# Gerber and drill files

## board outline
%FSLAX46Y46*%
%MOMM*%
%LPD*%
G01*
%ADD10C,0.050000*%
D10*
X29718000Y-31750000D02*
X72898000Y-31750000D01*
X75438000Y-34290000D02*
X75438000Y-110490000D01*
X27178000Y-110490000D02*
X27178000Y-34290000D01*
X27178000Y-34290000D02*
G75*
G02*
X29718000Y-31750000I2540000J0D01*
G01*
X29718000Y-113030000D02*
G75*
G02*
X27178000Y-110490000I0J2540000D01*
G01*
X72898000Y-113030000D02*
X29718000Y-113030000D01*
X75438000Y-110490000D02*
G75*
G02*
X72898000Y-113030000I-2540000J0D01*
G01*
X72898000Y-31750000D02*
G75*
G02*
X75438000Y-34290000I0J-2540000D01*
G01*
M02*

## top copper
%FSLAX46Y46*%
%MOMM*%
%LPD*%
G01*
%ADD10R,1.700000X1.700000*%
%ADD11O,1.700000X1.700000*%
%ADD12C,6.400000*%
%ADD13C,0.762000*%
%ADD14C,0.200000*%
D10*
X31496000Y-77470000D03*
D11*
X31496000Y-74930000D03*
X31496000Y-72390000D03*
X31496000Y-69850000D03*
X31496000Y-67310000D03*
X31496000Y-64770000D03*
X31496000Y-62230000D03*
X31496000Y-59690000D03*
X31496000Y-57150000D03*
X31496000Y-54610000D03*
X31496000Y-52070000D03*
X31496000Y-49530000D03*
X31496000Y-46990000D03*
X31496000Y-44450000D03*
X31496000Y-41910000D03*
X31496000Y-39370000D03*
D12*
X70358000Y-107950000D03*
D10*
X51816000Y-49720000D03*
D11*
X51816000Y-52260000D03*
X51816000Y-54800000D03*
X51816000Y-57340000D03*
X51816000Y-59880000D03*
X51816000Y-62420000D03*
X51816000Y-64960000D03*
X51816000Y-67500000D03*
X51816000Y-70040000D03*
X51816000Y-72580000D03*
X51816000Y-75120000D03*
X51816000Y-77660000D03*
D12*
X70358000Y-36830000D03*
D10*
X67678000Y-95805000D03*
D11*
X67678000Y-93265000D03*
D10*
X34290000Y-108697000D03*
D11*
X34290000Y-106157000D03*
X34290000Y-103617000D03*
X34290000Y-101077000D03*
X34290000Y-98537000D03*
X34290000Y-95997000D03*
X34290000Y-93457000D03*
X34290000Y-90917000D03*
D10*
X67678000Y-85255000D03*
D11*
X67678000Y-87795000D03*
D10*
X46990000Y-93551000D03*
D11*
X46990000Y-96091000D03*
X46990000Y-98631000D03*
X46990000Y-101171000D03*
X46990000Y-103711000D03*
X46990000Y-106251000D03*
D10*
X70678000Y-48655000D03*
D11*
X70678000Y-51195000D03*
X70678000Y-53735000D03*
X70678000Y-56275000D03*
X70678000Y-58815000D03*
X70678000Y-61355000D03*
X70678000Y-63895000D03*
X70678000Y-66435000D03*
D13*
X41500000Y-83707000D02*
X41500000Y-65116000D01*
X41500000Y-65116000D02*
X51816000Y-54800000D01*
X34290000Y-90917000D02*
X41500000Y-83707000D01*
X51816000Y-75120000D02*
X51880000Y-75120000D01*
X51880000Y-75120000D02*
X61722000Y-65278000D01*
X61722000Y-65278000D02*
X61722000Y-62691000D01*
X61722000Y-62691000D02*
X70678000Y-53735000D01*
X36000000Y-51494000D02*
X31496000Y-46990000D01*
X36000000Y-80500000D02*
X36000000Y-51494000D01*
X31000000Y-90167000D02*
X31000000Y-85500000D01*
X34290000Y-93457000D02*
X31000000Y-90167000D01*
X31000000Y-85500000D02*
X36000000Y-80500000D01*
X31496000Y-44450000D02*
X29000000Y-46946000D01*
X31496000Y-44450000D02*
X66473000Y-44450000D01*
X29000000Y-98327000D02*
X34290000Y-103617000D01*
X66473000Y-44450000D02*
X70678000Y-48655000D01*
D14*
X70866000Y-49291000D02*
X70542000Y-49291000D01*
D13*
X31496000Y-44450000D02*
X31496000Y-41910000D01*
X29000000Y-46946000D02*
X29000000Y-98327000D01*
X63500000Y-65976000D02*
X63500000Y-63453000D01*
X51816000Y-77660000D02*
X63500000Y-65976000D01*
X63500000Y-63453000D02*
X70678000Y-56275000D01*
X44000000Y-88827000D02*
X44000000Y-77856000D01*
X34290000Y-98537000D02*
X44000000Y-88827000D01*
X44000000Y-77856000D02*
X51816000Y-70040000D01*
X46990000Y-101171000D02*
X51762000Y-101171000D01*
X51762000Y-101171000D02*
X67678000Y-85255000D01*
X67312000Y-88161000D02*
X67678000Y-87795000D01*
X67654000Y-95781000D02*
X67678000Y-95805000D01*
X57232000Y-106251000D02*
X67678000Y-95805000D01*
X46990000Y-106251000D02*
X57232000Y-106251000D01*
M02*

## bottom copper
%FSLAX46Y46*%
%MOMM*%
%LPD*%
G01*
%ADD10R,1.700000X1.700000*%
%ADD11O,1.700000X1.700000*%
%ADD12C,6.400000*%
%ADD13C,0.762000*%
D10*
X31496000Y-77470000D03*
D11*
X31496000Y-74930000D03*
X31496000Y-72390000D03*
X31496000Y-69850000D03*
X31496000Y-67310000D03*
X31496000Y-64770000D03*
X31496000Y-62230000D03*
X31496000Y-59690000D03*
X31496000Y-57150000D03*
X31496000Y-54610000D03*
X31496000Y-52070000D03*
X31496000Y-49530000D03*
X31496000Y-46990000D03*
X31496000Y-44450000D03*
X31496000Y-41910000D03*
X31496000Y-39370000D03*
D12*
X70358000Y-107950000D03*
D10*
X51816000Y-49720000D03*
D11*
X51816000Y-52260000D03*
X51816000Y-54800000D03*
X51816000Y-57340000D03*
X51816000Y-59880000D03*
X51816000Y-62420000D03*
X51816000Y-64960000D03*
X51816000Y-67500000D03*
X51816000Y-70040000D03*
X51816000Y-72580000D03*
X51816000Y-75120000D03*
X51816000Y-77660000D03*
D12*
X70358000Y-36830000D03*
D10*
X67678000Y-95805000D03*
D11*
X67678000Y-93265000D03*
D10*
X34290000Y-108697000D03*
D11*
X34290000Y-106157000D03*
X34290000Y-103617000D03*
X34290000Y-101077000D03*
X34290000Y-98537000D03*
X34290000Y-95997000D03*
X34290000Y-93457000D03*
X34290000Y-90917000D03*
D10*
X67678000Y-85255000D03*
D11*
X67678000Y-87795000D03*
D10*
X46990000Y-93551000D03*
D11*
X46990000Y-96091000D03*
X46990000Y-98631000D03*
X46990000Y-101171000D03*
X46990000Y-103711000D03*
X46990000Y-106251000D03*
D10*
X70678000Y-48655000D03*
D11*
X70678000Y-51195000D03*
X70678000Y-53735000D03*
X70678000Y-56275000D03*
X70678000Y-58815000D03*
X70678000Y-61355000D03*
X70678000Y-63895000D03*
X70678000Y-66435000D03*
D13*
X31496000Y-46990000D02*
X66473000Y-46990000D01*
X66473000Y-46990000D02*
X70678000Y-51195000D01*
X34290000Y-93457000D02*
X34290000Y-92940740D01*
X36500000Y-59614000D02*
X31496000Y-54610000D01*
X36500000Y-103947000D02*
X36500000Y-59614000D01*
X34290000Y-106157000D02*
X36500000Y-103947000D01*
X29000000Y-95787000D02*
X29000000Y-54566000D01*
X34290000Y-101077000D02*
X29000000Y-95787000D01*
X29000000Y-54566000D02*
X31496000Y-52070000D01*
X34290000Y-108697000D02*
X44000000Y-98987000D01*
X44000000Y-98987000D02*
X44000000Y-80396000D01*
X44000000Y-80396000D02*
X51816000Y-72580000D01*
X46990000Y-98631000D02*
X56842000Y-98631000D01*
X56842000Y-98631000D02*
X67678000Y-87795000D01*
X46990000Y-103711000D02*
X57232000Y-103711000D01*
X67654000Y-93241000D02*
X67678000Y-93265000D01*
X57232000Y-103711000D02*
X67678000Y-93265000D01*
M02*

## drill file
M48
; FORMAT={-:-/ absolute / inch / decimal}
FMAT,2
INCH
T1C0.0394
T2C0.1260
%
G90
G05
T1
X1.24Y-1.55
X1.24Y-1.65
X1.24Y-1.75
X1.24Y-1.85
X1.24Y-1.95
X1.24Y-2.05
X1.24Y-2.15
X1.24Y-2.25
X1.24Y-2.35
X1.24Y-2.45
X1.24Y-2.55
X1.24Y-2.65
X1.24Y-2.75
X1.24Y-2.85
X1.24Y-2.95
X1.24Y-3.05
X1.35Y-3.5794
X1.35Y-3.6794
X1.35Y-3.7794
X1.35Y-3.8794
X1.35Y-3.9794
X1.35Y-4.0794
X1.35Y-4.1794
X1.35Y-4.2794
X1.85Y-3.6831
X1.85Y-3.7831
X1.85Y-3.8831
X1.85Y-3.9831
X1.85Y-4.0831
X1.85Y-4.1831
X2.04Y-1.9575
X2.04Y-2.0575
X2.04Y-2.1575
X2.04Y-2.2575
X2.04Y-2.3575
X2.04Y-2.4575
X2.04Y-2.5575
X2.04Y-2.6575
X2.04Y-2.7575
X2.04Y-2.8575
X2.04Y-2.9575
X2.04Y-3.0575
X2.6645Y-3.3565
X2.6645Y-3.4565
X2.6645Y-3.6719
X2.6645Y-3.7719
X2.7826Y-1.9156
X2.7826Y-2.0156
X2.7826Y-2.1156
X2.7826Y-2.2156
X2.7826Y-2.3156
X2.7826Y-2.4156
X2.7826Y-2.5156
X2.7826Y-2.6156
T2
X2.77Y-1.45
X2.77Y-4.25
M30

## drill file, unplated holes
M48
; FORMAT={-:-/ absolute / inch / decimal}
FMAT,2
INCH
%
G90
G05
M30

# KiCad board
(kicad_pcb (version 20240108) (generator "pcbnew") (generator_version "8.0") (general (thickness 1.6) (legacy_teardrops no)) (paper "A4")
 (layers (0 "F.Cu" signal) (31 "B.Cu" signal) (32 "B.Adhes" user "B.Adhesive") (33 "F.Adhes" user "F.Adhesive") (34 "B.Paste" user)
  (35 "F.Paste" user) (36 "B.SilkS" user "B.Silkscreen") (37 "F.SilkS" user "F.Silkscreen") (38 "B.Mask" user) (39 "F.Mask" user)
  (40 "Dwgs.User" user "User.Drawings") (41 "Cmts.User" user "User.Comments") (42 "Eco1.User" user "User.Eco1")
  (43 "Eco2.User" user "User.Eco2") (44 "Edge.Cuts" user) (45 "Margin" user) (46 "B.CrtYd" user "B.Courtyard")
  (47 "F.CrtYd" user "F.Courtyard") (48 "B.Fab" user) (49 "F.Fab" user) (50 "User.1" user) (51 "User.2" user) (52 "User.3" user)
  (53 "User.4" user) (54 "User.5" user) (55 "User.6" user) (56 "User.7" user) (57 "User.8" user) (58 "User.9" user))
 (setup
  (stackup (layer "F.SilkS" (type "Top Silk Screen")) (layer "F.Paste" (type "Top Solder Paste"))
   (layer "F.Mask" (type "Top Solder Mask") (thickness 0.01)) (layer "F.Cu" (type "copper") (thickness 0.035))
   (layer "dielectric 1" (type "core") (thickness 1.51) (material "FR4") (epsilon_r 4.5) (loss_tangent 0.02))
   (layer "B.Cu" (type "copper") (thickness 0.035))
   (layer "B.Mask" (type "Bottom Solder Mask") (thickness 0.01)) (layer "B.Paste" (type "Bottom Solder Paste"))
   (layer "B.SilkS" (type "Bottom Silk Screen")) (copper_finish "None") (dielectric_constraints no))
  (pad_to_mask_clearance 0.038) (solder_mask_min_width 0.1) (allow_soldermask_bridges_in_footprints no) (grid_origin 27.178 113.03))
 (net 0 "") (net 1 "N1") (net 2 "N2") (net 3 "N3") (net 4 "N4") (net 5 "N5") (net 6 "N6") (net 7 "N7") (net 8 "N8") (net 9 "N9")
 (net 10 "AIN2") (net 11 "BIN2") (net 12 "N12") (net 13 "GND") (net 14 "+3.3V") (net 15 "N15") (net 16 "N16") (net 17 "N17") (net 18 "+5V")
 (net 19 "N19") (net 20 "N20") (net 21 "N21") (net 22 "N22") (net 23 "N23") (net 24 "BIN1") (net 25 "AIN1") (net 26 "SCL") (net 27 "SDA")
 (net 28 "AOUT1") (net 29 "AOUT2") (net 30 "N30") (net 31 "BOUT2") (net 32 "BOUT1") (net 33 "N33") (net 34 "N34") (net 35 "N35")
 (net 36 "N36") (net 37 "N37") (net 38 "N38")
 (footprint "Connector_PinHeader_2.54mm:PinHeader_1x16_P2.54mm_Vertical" (layer "F.Cu") (at 31.496 77.47 180)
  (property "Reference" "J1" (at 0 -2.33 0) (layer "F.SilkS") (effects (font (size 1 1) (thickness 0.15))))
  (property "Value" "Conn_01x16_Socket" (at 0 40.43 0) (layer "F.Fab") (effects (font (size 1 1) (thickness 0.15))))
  (pad "1" thru_hole rect (at 0 0 180) (size 1.7 1.7) (drill 1) (layers "*.Cu" "*.Mask") (remove_unused_layers no) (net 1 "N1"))
  (pad "2" thru_hole oval (at 0 2.54 180) (size 1.7 1.7) (drill 1) (layers "*.Cu" "*.Mask") (remove_unused_layers no) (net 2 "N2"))
  (pad "3" thru_hole oval (at 0 5.08 180) (size 1.7 1.7) (drill 1) (layers "*.Cu" "*.Mask") (remove_unused_layers no) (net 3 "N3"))
  (pad "4" thru_hole oval (at 0 7.62 180) (size 1.7 1.7) (drill 1) (layers "*.Cu" "*.Mask") (remove_unused_layers no) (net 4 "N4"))
  (pad "5" thru_hole oval (at 0 10.16 180) (size 1.7 1.7) (drill 1) (layers "*.Cu" "*.Mask") (remove_unused_layers no) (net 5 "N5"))
  (pad "6" thru_hole oval (at 0 12.7 180) (size 1.7 1.7) (drill 1) (layers "*.Cu" "*.Mask") (remove_unused_layers no) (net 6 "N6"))
  (pad "7" thru_hole oval (at 0 15.24 180) (size 1.7 1.7) (drill 1) (layers "*.Cu" "*.Mask") (remove_unused_layers no) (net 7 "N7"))
  (pad "8" thru_hole oval (at 0 17.78 180) (size 1.7 1.7) (drill 1) (layers "*.Cu" "*.Mask") (remove_unused_layers no) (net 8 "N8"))
  (pad "9" thru_hole oval (at 0 20.32 180) (size 1.7 1.7) (drill 1) (layers "*.Cu" "*.Mask") (remove_unused_layers no) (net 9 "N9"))
  (pad "10" thru_hole oval (at 0 22.86 180) (size 1.7 1.7) (drill 1) (layers "*.Cu" "*.Mask") (remove_unused_layers no) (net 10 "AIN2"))
  (pad "11" thru_hole oval (at 0 25.4 180) (size 1.7 1.7) (drill 1) (layers "*.Cu" "*.Mask") (remove_unused_layers no) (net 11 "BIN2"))
  (pad "12" thru_hole oval (at 0 27.94 180) (size 1.7 1.7) (drill 1) (layers "*.Cu" "*.Mask") (remove_unused_layers no) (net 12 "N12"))
  (pad "13" thru_hole oval (at 0 30.48 180) (size 1.7 1.7) (drill 1) (layers "*.Cu" "*.Mask") (remove_unused_layers no) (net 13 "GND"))
  (pad "14" thru_hole oval (at 0 33.02 180) (size 1.7 1.7) (drill 1) (layers "*.Cu" "*.Mask") (remove_unused_layers no) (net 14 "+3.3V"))
  (pad "15" thru_hole oval (at 0 35.56 180) (size 1.7 1.7) (drill 1) (layers "*.Cu" "*.Mask") (remove_unused_layers no) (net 14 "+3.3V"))
  (pad "16" thru_hole oval (at 0 38.1 180) (size 1.7 1.7) (drill 1) (layers "*.Cu" "*.Mask") (remove_unused_layers no) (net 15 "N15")))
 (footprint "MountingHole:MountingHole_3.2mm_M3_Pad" (layer "F.Cu") (at 70.358 107.95)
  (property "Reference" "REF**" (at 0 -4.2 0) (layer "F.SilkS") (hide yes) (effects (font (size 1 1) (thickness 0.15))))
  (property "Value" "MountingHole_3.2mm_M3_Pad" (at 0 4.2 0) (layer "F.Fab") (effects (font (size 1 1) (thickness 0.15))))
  (pad "1" thru_hole circle (at 0 0) (size 6.4 6.4) (drill 3.2) (layers "*.Cu" "*.Mask") (remove_unused_layers no)))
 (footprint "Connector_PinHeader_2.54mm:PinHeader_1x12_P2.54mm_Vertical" (layer "F.Cu") (at 51.816 49.72)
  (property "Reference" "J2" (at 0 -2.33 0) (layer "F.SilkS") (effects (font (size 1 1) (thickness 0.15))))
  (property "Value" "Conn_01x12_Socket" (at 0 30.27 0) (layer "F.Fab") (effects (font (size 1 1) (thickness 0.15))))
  (pad "1" thru_hole rect (at 0 0) (size 1.7 1.7) (drill 1) (layers "*.Cu" "*.Mask") (remove_unused_layers no) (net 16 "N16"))
  (pad "2" thru_hole oval (at 0 2.54) (size 1.7 1.7) (drill 1) (layers "*.Cu" "*.Mask") (remove_unused_layers no) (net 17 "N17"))
  (pad "3" thru_hole oval (at 0 5.08) (size 1.7 1.7) (drill 1) (layers "*.Cu" "*.Mask") (remove_unused_layers no) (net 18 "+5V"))
  (pad "4" thru_hole oval (at 0 7.62) (size 1.7 1.7) (drill 1) (layers "*.Cu" "*.Mask") (remove_unused_layers no) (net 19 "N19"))
  (pad "5" thru_hole oval (at 0 10.16) (size 1.7 1.7) (drill 1) (layers "*.Cu" "*.Mask") (remove_unused_layers no) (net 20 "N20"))
  (pad "6" thru_hole oval (at 0 12.7) (size 1.7 1.7) (drill 1) (layers "*.Cu" "*.Mask") (remove_unused_layers no) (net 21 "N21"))
  (pad "7" thru_hole oval (at 0 15.24) (size 1.7 1.7) (drill 1) (layers "*.Cu" "*.Mask") (remove_unused_layers no) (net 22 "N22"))
  (pad "8" thru_hole oval (at 0 17.78) (size 1.7 1.7) (drill 1) (layers "*.Cu" "*.Mask") (remove_unused_layers no) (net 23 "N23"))
  (pad "9" thru_hole oval (at 0 20.32) (size 1.7 1.7) (drill 1) (layers "*.Cu" "*.Mask") (remove_unused_layers no) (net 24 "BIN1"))
  (pad "10" thru_hole oval (at 0 22.86) (size 1.7 1.7) (drill 1) (layers "*.Cu" "*.Mask") (remove_unused_layers no) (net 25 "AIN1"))
  (pad "11" thru_hole oval (at 0 25.4) (size 1.7 1.7) (drill 1) (layers "*.Cu" "*.Mask") (remove_unused_layers no) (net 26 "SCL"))
  (pad "12" thru_hole oval (at 0 27.94) (size 1.7 1.7) (drill 1) (layers "*.Cu" "*.Mask") (remove_unused_layers no) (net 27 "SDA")))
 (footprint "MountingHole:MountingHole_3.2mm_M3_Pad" (layer "F.Cu") (at 70.358 36.83)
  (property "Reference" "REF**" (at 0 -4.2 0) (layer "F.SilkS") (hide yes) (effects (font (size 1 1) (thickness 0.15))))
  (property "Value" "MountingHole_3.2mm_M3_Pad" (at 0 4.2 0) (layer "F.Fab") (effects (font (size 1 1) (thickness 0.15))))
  (pad "1" thru_hole circle (at 0 0) (size 6.4 6.4) (drill 3.2) (layers "*.Cu" "*.Mask") (remove_unused_layers no)))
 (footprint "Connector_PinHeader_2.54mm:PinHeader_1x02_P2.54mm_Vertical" (layer "F.Cu") (at 67.678 95.805 180)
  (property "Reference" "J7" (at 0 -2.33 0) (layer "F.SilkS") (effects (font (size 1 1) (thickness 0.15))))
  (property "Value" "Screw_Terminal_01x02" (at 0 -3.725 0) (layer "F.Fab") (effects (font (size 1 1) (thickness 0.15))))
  (pad "1" thru_hole rect (at 0 0 180) (size 1.7 1.7) (drill 1) (layers "*.Cu" "*.Mask") (remove_unused_layers no) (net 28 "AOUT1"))
  (pad "2" thru_hole oval (at 0 2.54 180) (size 1.7 1.7) (drill 1) (layers "*.Cu" "*.Mask") (remove_unused_layers no) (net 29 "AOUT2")))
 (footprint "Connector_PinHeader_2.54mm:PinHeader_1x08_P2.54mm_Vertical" (layer "F.Cu") (at 34.29 108.697 180)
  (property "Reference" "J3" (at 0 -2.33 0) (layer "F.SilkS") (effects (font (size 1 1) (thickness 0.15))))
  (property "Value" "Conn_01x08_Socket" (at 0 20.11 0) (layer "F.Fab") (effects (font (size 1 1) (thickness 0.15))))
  (pad "1" thru_hole rect (at 0 0 180) (size 1.7 1.7) (drill 1) (layers "*.Cu" "*.Mask") (remove_unused_layers no) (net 25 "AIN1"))
  (pad "2" thru_hole oval (at 0 2.54 180) (size 1.7 1.7) (drill 1) (layers "*.Cu" "*.Mask") (remove_unused_layers no) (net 10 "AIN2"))
  (pad "3" thru_hole oval (at 0 5.08 180) (size 1.7 1.7) (drill 1) (layers "*.Cu" "*.Mask") (remove_unused_layers no) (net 14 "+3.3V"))
  (pad "4" thru_hole oval (at 0 7.62 180) (size 1.7 1.7) (drill 1) (layers "*.Cu" "*.Mask") (remove_unused_layers no) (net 11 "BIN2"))
  (pad "5" thru_hole oval (at 0 10.16 180) (size 1.7 1.7) (drill 1) (layers "*.Cu" "*.Mask") (remove_unused_layers no) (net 24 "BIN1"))
  (pad "6" thru_hole oval (at 0 12.7 180) (size 1.7 1.7) (drill 1) (layers "*.Cu" "*.Mask") (remove_unused_layers no) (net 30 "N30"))
  (pad "7" thru_hole oval (at 0 15.24 180) (size 1.7 1.7) (drill 1) (layers "*.Cu" "*.Mask") (remove_unused_layers no) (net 13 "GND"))
  (pad "8" thru_hole oval (at 0 17.78 180) (size 1.7 1.7) (drill 1) (layers "*.Cu" "*.Mask") (remove_unused_layers no) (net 18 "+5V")))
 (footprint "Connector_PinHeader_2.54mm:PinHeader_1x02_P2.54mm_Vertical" (layer "F.Cu") (at 67.678 85.255)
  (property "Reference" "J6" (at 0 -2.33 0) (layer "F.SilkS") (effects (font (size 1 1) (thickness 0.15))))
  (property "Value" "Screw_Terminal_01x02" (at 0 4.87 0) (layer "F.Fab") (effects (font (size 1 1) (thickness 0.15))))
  (pad "1" thru_hole rect (at 0 0) (size 1.7 1.7) (drill 1) (layers "*.Cu" "*.Mask") (remove_unused_layers no) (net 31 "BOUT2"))
  (pad "2" thru_hole oval (at 0 2.54) (size 1.7 1.7) (drill 1) (layers "*.Cu" "*.Mask") (remove_unused_layers no) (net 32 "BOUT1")))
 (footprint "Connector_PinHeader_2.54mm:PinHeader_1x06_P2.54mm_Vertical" (layer "F.Cu") (at 46.99 93.551)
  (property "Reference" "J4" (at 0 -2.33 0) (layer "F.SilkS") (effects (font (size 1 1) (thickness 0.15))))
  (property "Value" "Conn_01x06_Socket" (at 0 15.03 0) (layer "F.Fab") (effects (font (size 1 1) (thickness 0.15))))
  (pad "1" thru_hole rect (at 0 0) (size 1.7 1.7) (drill 1) (layers "*.Cu" "*.Mask") (remove_unused_layers no) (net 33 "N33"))
  (pad "2" thru_hole oval (at 0 2.54) (size 1.7 1.7) (drill 1) (layers "*.Cu" "*.Mask") (remove_unused_layers no) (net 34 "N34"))
  (pad "3" thru_hole oval (at 0 5.08) (size 1.7 1.7) (drill 1) (layers "*.Cu" "*.Mask") (remove_unused_layers no) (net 32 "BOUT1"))
  (pad "4" thru_hole oval (at 0 7.62) (size 1.7 1.7) (drill 1) (layers "*.Cu" "*.Mask") (remove_unused_layers no) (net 31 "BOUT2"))
  (pad "5" thru_hole oval (at 0 10.16) (size 1.7 1.7) (drill 1) (layers "*.Cu" "*.Mask") (remove_unused_layers no) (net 29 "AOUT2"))
  (pad "6" thru_hole oval (at 0 12.7) (size 1.7 1.7) (drill 1) (layers "*.Cu" "*.Mask") (remove_unused_layers no) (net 28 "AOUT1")))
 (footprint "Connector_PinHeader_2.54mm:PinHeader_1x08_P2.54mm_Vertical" (layer "F.Cu") (at 70.678 48.655)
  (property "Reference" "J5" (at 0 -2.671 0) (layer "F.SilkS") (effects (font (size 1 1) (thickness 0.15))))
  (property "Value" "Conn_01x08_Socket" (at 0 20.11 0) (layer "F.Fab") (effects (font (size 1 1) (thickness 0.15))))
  (pad "1" thru_hole rect (at 0 0) (size 1.7 1.7) (drill 1) (layers "*.Cu" "*.Mask") (remove_unused_layers no) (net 14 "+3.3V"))
  (pad "2" thru_hole oval (at 0 2.54) (size 1.7 1.7) (drill 1) (layers "*.Cu" "*.Mask") (remove_unused_layers no) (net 13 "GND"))
  (pad "3" thru_hole oval (at 0 5.08) (size 1.7 1.7) (drill 1) (layers "*.Cu" "*.Mask") (remove_unused_layers no) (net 26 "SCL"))
  (pad "4" thru_hole oval (at 0 7.62) (size 1.7 1.7) (drill 1) (layers "*.Cu" "*.Mask") (remove_unused_layers no) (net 27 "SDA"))
  (pad "5" thru_hole oval (at 0 10.16) (size 1.7 1.7) (drill 1) (layers "*.Cu" "*.Mask") (remove_unused_layers no) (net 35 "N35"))
  (pad "6" thru_hole oval (at 0 12.7) (size 1.7 1.7) (drill 1) (layers "*.Cu" "*.Mask") (remove_unused_layers no) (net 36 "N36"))
  (pad "7" thru_hole oval (at 0 15.24) (size 1.7 1.7) (drill 1) (layers "*.Cu" "*.Mask") (remove_unused_layers no) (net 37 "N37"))
  (pad "8" thru_hole oval (at 0 17.78) (size 1.7 1.7) (drill 1) (layers "*.Cu" "*.Mask") (remove_unused_layers no) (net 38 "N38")))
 (gr_line (start 29.718 31.75) (end 72.898 31.75) (stroke (width 0.05) (type default)) (layer "Edge.Cuts"))
 (gr_line (start 75.438 34.29) (end 75.438 110.49) (stroke (width 0.05) (type default)) (layer "Edge.Cuts"))
 (gr_line (start 27.178 110.49) (end 27.178 34.29) (stroke (width 0.05) (type default)) (layer "Edge.Cuts"))
 (gr_arc (start 27.178 34.29) (mid 27.921949 32.493949) (end 29.718 31.75) (stroke (width 0.05) (type default)) (layer "Edge.Cuts"))
 (gr_arc (start 29.718 113.03) (mid 27.921949 112.286051) (end 27.178 110.49) (stroke (width 0.05) (type default)) (layer "Edge.Cuts"))
 (gr_line (start 72.898 113.03) (end 29.718 113.03) (stroke (width 0.05) (type default)) (layer "Edge.Cuts"))
 (gr_arc (start 75.438 110.49) (mid 74.694051 112.286051) (end 72.898 113.03) (stroke (width 0.05) (type default)) (layer "Edge.Cuts"))
 (gr_arc (start 72.898 31.75) (mid 74.694051 32.493949) (end 75.438 34.29) (stroke (width 0.05) (type default)) (layer "Edge.Cuts"))
 (segment (start 41.5 83.707) (end 41.5 65.116) (width 0.762) (layer "F.Cu") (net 18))
 (segment (start 41.5 65.116) (end 51.816 54.8) (width 0.762) (layer "F.Cu") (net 18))
 (segment (start 34.29 90.917) (end 41.5 83.707) (width 0.762) (layer "F.Cu") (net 18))
 (segment (start 51.816 75.12) (end 51.88 75.12) (width 0.762) (layer "F.Cu") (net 26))
 (segment (start 51.88 75.12) (end 61.722 65.278) (width 0.762) (layer "F.Cu") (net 26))
 (segment (start 61.722 65.278) (end 61.722 62.691) (width 0.762) (layer "F.Cu") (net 26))
 (segment (start 61.722 62.691) (end 70.678 53.735) (width 0.762) (layer "F.Cu") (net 26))
 (segment (start 36 51.494) (end 31.496 46.99) (width 0.762) (layer "F.Cu") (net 13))
 (segment (start 36 80.5) (end 36 51.494) (width 0.762) (layer "F.Cu") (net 13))
 (segment (start 31 90.167) (end 31 85.5) (width 0.762) (layer "F.Cu") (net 13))
 (segment (start 34.29 93.457) (end 31 90.167) (width 0.762) (layer "F.Cu") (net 13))
 (segment (start 31 85.5) (end 36 80.5) (width 0.762) (layer "F.Cu") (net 13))
 (segment (start 31.496 46.99) (end 66.473 46.99) (width 0.762) (layer "B.Cu") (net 13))
 (segment (start 66.473 46.99) (end 70.678 51.195) (width 0.762) (layer "B.Cu") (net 13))
 (segment (start 34.29 93.457) (end 34.29 92.94074) (width 0.762) (layer "B.Cu") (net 13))
 (segment (start 31.496 44.45) (end 29 46.946) (width 0.762) (layer "F.Cu") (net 14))
 (segment (start 31.496 44.45) (end 66.473 44.45) (width 0.762) (layer "F.Cu") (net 14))
 (segment (start 29 98.327) (end 34.29 103.617) (width 0.762) (layer "F.Cu") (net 14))
 (segment (start 66.473 44.45) (end 70.678 48.655) (width 0.762) (layer "F.Cu") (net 14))
 (segment (start 70.866 49.291) (end 70.542 49.291) (width 0.2) (layer "F.Cu") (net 14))
 (segment (start 31.496 44.45) (end 31.496 41.91) (width 0.762) (layer "F.Cu") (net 14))
 (segment (start 29 46.946) (end 29 98.327) (width 0.762) (layer "F.Cu") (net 14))
 (segment (start 63.5 65.976) (end 63.5 63.453) (width 0.762) (layer "F.Cu") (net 27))
 (segment (start 51.816 77.66) (end 63.5 65.976) (width 0.762) (layer "F.Cu") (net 27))
 (segment (start 63.5 63.453) (end 70.678 56.275) (width 0.762) (layer "F.Cu") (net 27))
 (segment (start 36.5 59.614) (end 31.496 54.61) (width 0.762) (layer "B.Cu") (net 10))
 (segment (start 36.5 103.947) (end 36.5 59.614) (width 0.762) (layer "B.Cu") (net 10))
 (segment (start 34.29 106.157) (end 36.5 103.947) (width 0.762) (layer "B.Cu") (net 10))
 (segment (start 29 95.787) (end 29 54.566) (width 0.762) (layer "B.Cu") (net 11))
 (segment (start 34.29 101.077) (end 29 95.787) (width 0.762) (layer "B.Cu") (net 11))
 (segment (start 29 54.566) (end 31.496 52.07) (width 0.762) (layer "B.Cu") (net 11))
 (segment (start 34.29 108.697) (end 44 98.987) (width 0.762) (layer "B.Cu") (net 25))
 (segment (start 44 98.987) (end 44 80.396) (width 0.762) (layer "B.Cu") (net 25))
 (segment (start 44 80.396) (end 51.816 72.58) (width 0.762) (layer "B.Cu") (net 25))
 (segment (start 44 88.827) (end 44 77.856) (width 0.762) (layer "F.Cu") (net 24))
 (segment (start 34.29 98.537) (end 44 88.827) (width 0.762) (layer "F.Cu") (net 24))
 (segment (start 44 77.856) (end 51.816 70.04) (width 0.762) (layer "F.Cu") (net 24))
 (segment (start 46.99 101.171) (end 51.762 101.171) (width 0.762) (layer "F.Cu") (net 31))
 (segment (start 51.762 101.171) (end 67.678 85.255) (width 0.762) (layer "F.Cu") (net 31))
 (segment (start 67.312 88.161) (end 67.678 87.795) (width 0.762) (layer "F.Cu") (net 32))
 (segment (start 46.99 98.631) (end 56.842 98.631) (width 0.762) (layer "B.Cu") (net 32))
 (segment (start 56.842 98.631) (end 67.678 87.795) (width 0.762) (layer "B.Cu") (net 32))
 (segment (start 46.99 103.711) (end 57.232 103.711) (width 0.762) (layer "B.Cu") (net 29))
 (segment (start 67.654 93.241) (end 67.678 93.265) (width 0.762) (layer "B.Cu") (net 29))
 (segment (start 57.232 103.711) (end 67.678 93.265) (width 0.762) (layer "B.Cu") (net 29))
 (segment (start 67.654 95.781) (end 67.678 95.805) (width 0.762) (layer "F.Cu") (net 28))
 (segment (start 57.232 106.251) (end 67.678 95.805) (width 0.762) (layer "F.Cu") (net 28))
 (segment (start 46.99 106.251) (end 57.232 106.251) (width 0.762) (layer "F.Cu") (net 28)))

